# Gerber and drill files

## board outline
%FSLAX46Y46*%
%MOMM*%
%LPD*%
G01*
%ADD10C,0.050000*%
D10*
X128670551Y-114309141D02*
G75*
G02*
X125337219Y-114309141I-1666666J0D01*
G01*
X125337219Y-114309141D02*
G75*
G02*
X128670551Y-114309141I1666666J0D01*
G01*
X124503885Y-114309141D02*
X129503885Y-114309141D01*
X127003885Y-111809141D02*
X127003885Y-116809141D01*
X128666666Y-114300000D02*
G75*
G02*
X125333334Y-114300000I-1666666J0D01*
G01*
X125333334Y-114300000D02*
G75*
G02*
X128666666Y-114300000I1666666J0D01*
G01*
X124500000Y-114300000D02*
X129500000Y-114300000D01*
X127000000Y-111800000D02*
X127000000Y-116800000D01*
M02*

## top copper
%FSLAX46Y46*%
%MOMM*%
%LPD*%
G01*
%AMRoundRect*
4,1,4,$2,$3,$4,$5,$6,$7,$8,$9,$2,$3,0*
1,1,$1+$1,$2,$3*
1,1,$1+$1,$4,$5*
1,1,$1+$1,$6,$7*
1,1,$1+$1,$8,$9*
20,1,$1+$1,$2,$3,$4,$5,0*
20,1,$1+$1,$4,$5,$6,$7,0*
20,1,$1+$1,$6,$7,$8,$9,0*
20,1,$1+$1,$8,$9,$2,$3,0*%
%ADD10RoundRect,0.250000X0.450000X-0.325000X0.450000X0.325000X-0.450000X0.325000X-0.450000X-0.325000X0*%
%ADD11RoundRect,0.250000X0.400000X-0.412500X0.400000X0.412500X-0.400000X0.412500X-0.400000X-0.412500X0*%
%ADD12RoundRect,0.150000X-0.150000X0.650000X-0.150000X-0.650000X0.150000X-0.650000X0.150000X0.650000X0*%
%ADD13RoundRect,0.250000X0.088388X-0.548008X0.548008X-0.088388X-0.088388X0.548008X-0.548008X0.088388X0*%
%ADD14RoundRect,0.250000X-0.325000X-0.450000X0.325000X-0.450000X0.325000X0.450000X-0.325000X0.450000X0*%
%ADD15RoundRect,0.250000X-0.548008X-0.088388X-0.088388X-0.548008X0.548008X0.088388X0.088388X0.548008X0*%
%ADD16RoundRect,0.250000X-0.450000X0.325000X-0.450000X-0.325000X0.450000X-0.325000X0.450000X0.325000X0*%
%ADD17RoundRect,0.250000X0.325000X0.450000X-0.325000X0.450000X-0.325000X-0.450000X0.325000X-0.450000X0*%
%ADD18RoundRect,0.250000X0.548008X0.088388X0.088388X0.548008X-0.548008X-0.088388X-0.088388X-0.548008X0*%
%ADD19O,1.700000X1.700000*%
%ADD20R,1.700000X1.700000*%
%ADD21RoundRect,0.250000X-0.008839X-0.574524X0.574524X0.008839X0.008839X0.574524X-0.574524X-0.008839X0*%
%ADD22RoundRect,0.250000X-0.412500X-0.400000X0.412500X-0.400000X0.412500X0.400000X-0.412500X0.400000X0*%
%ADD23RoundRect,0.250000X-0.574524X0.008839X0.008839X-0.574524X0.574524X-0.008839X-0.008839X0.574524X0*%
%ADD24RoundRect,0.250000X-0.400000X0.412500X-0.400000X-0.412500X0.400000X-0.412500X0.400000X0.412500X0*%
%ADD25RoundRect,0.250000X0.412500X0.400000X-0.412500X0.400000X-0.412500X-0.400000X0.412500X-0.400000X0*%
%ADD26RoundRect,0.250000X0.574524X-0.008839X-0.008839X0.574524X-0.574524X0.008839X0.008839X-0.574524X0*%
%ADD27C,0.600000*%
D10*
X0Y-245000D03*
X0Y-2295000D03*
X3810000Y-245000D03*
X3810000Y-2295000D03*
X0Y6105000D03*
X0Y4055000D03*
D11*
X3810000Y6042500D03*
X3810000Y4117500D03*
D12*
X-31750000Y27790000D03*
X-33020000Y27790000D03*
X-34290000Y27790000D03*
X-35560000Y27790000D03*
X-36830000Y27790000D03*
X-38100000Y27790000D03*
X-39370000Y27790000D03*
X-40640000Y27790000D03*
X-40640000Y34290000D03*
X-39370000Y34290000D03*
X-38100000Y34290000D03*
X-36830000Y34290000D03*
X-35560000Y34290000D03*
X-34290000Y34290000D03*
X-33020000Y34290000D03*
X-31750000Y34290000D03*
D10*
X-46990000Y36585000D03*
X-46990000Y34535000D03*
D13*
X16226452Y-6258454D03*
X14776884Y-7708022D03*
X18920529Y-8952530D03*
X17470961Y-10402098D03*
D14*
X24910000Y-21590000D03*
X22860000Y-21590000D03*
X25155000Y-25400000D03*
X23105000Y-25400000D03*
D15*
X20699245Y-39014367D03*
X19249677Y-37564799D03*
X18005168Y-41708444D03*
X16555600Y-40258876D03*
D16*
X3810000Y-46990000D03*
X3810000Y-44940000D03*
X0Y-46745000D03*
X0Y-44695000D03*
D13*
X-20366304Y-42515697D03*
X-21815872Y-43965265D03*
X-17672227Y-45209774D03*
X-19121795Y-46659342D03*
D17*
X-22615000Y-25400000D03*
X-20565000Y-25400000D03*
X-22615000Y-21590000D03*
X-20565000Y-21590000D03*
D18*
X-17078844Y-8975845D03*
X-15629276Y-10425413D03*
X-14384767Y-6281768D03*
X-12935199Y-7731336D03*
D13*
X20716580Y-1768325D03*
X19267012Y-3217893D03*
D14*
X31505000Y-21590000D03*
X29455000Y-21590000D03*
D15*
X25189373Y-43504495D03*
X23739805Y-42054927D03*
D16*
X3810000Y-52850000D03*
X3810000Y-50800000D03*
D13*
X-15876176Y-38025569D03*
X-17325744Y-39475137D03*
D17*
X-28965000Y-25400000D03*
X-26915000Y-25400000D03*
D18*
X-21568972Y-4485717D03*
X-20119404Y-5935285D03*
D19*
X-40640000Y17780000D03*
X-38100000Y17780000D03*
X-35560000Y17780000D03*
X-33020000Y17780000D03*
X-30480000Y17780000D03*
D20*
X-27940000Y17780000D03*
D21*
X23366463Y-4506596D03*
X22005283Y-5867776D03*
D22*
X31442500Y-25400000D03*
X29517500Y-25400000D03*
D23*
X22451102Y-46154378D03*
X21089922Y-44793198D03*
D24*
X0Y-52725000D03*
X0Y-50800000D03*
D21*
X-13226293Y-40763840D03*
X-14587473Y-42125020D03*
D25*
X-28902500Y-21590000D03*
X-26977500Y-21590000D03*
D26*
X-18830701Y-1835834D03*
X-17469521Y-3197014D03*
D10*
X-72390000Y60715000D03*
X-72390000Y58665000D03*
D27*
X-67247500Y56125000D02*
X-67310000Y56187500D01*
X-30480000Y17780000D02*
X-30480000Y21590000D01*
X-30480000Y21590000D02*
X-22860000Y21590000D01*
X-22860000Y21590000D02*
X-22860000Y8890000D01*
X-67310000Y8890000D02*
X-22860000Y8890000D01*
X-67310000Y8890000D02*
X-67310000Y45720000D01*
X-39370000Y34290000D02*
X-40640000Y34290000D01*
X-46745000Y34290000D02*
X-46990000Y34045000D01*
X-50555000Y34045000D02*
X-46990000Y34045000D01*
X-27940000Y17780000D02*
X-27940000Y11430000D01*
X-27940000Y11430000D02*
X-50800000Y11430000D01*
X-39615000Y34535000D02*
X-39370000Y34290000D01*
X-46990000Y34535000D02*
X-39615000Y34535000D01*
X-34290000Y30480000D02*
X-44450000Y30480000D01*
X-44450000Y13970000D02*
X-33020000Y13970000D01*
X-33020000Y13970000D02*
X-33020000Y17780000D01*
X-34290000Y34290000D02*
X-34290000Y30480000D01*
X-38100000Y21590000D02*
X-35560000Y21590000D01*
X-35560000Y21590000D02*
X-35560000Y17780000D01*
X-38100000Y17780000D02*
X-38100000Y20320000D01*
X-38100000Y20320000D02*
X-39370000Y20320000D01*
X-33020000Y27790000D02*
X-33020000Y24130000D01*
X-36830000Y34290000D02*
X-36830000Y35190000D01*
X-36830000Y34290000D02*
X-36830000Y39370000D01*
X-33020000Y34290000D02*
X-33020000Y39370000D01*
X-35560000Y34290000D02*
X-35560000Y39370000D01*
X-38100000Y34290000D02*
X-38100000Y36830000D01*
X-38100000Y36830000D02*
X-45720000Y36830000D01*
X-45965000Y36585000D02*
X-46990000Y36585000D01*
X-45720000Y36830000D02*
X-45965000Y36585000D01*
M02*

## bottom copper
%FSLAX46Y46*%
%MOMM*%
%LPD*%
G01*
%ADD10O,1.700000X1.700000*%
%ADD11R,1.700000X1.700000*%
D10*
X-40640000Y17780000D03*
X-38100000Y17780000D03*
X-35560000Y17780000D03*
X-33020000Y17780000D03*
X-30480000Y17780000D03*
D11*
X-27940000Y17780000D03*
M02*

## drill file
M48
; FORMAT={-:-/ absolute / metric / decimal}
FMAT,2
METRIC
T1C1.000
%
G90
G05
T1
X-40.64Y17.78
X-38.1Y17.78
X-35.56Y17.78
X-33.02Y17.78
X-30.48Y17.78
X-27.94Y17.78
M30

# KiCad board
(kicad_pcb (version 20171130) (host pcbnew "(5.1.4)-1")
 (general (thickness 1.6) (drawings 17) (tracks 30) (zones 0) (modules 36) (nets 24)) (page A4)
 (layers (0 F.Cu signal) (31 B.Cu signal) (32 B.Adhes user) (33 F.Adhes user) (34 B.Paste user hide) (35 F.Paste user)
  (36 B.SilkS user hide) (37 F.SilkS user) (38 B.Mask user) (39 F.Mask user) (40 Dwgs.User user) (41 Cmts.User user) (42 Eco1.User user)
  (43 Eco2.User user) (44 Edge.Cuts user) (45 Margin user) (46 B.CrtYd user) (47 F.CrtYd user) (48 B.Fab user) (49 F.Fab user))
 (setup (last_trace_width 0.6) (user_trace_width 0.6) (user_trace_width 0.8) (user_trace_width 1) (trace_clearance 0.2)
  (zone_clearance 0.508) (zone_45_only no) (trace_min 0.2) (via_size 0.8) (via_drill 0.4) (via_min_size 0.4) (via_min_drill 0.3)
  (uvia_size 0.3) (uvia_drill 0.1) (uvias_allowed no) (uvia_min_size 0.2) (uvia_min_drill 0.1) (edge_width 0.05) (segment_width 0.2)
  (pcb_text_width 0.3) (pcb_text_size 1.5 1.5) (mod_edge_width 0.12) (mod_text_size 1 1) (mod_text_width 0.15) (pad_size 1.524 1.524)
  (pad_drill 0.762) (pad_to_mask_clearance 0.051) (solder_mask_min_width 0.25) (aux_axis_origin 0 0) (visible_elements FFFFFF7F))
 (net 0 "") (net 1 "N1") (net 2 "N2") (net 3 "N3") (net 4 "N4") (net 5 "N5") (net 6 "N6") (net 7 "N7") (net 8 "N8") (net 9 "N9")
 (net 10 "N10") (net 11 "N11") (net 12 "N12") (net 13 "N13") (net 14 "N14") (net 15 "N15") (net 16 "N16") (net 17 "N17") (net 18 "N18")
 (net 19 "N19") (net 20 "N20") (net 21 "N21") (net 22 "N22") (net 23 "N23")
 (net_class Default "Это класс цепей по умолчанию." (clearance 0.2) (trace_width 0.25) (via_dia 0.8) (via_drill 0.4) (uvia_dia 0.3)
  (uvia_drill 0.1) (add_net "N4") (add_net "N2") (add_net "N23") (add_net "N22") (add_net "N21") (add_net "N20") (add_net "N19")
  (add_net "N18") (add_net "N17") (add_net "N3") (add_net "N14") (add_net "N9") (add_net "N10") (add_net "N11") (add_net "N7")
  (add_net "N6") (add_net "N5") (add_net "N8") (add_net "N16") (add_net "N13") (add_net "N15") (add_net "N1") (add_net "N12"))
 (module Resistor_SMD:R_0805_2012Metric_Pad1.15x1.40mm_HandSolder (layer F.Cu) (at 0 1.27 90)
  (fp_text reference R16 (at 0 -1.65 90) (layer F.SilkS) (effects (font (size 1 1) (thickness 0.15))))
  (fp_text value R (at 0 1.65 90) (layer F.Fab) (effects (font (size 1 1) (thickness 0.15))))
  (pad 2 smd roundrect (at 1.025 0 90) (size 1.15 1.4) (layers F.Cu F.Paste F.Mask) (roundrect_rratio 0.217391) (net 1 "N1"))
  (pad 1 smd roundrect (at -1.025 0 90) (size 1.15 1.4) (layers F.Cu F.Paste F.Mask) (roundrect_rratio 0.217391) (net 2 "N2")))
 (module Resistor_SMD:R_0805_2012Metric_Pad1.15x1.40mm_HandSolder (layer F.Cu) (at 3.81 1.27 90)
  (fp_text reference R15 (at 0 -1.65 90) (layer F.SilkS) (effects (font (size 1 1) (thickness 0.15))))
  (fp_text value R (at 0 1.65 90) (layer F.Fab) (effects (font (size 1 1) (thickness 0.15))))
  (pad 2 smd roundrect (at 1.025 0 90) (size 1.15 1.4) (layers F.Cu F.Paste F.Mask) (roundrect_rratio 0.217391) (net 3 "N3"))
  (pad 1 smd roundrect (at -1.025 0 90) (size 1.15 1.4) (layers F.Cu F.Paste F.Mask) (roundrect_rratio 0.217391) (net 2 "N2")))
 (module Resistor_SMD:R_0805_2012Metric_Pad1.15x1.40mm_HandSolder (layer F.Cu) (at 0 -5.08 90)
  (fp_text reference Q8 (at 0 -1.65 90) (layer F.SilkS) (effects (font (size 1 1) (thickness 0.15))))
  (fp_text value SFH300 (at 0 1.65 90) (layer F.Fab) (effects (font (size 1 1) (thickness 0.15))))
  (pad 2 smd roundrect (at 1.025 0 90) (size 1.15 1.4) (layers F.Cu F.Paste F.Mask) (roundrect_rratio 0.217391) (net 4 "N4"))
  (pad 1 smd roundrect (at -1.025 0 90) (size 1.15 1.4) (layers F.Cu F.Paste F.Mask) (roundrect_rratio 0.217391) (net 1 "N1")))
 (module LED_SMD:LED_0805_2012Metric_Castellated (layer F.Cu) (at 3.81 -5.08 90)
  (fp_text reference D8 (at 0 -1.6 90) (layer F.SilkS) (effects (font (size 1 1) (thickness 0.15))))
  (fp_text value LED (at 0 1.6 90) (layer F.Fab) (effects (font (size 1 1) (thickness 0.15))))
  (pad 2 smd roundrect (at 0.9625 0 90) (size 1.325 1.3) (layers F.Cu F.Paste F.Mask) (roundrect_rratio 0.192308) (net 4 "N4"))
  (pad 1 smd roundrect (at -0.9625 0 90) (size 1.325 1.3) (layers F.Cu F.Paste F.Mask) (roundrect_rratio 0.192308) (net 3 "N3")))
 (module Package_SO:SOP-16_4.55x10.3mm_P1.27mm (layer F.Cu) (at -36.195 -31.04 270)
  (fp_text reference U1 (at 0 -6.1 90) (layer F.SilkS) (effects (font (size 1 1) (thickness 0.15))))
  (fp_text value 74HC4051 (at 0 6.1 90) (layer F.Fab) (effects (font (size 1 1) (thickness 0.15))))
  (pad 16 smd roundrect (at 3.25 -4.445 270) (size 1.6 0.6) (layers F.Cu F.Paste F.Mask) (roundrect_rratio 0.25) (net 4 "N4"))
  (pad 15 smd roundrect (at 3.25 -3.175 270) (size 1.6 0.6) (layers F.Cu F.Paste F.Mask) (roundrect_rratio 0.25) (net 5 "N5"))
  (pad 14 smd roundrect (at 3.25 -1.905 270) (size 1.6 0.6) (layers F.Cu F.Paste F.Mask) (roundrect_rratio 0.25) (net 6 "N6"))
  (pad 13 smd roundrect (at 3.25 -0.635 270) (size 1.6 0.6) (layers F.Cu F.Paste F.Mask) (roundrect_rratio 0.25) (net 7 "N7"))
  (pad 12 smd roundrect (at 3.25 0.635 270) (size 1.6 0.6) (layers F.Cu F.Paste F.Mask) (roundrect_rratio 0.25) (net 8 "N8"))
  (pad 11 smd roundrect (at 3.25 1.905 270) (size 1.6 0.6) (layers F.Cu F.Paste F.Mask) (roundrect_rratio 0.25) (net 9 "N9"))
  (pad 10 smd roundrect (at 3.25 3.175 270) (size 1.6 0.6) (layers F.Cu F.Paste F.Mask) (roundrect_rratio 0.25) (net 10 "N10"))
  (pad 9 smd roundrect (at 3.25 4.445 270) (size 1.6 0.6) (layers F.Cu F.Paste F.Mask) (roundrect_rratio 0.25) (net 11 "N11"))
  (pad 8 smd roundrect (at -3.25 4.445 270) (size 1.6 0.6) (layers F.Cu F.Paste F.Mask) (roundrect_rratio 0.25) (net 2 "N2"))
  (pad 7 smd roundrect (at -3.25 3.175 270) (size 1.6 0.6) (layers F.Cu F.Paste F.Mask) (roundrect_rratio 0.25) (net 2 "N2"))
  (pad 6 smd roundrect (at -3.25 1.905 270) (size 1.6 0.6) (layers F.Cu F.Paste F.Mask) (roundrect_rratio 0.25) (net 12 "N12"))
  (pad 5 smd roundrect (at -3.25 0.635 270) (size 1.6 0.6) (layers F.Cu F.Paste F.Mask) (roundrect_rratio 0.25) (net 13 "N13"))
  (pad 4 smd roundrect (at -3.25 -0.635 270) (size 1.6 0.6) (layers F.Cu F.Paste F.Mask) (roundrect_rratio 0.25) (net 1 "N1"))
  (pad 3 smd roundrect (at -3.25 -1.905 270) (size 1.6 0.6) (layers F.Cu F.Paste F.Mask) (roundrect_rratio 0.25) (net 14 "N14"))
  (pad 2 smd roundrect (at -3.25 -3.175 270) (size 1.6 0.6) (layers F.Cu F.Paste F.Mask) (roundrect_rratio 0.25) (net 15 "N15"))
  (pad 1 smd roundrect (at -3.25 -4.445 270) (size 1.6 0.6) (layers F.Cu F.Paste F.Mask) (roundrect_rratio 0.25) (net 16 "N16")))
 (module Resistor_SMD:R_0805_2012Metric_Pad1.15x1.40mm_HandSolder (layer F.Cu) (at -46.99 -35.56 90)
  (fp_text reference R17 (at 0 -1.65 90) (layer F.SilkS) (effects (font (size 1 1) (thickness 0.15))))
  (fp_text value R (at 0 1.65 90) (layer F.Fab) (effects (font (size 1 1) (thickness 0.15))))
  (pad 2 smd roundrect (at 1.025 0 90) (size 1.15 1.4) (layers F.Cu F.Paste F.Mask) (roundrect_rratio 0.217391) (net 12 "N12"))
  (pad 1 smd roundrect (at -1.025 0 90) (size 1.15 1.4) (layers F.Cu F.Paste F.Mask) (roundrect_rratio 0.217391) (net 2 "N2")))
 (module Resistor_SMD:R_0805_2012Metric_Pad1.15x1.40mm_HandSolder (layer F.Cu) (at 15.501668 6.983238 45)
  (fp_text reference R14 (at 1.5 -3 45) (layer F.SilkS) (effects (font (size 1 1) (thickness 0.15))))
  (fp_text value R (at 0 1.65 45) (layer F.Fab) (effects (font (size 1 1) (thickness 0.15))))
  (pad 2 smd roundrect (at 1.025 0 45) (size 1.15 1.4) (layers F.Cu F.Paste F.Mask) (roundrect_rratio 0.217391) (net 15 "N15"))
  (pad 1 smd roundrect (at -1.025 0 45) (size 1.15 1.4) (layers F.Cu F.Paste F.Mask) (roundrect_rratio 0.217391) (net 2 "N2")))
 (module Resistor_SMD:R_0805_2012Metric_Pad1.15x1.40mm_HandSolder (layer F.Cu) (at 18.195745 9.677314 45)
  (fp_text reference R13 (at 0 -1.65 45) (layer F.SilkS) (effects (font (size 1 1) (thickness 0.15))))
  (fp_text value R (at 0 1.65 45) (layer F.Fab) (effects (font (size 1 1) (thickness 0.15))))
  (pad 2 smd roundrect (at 1.025 0 45) (size 1.15 1.4) (layers F.Cu F.Paste F.Mask) (roundrect_rratio 0.217391) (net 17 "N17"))
  (pad 1 smd roundrect (at -1.025 0 45) (size 1.15 1.4) (layers F.Cu F.Paste F.Mask) (roundrect_rratio 0.217391) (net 2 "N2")))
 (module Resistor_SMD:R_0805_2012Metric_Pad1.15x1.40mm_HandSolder (layer F.Cu) (at 23.885 21.59)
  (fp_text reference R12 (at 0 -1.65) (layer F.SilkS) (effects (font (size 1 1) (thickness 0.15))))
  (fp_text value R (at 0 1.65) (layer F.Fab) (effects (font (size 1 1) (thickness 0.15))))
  (pad 2 smd roundrect (at 1.025 0) (size 1.15 1.4) (layers F.Cu F.Paste F.Mask) (roundrect_rratio 0.217391) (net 13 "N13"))
  (pad 1 smd roundrect (at -1.025 0) (size 1.15 1.4) (layers F.Cu F.Paste F.Mask) (roundrect_rratio 0.217391) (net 2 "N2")))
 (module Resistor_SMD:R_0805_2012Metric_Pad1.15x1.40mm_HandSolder (layer F.Cu) (at 24.13 25.4)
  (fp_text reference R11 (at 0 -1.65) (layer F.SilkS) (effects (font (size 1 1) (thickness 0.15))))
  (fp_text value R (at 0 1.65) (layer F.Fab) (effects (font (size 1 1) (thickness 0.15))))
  (pad 2 smd roundrect (at 1.025 0) (size 1.15 1.4) (layers F.Cu F.Paste F.Mask) (roundrect_rratio 0.217391) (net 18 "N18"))
  (pad 1 smd roundrect (at -1.025 0) (size 1.15 1.4) (layers F.Cu F.Paste F.Mask) (roundrect_rratio 0.217391) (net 2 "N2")))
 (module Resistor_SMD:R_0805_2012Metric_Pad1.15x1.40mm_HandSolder (layer F.Cu) (at 19.974461 38.289583 315)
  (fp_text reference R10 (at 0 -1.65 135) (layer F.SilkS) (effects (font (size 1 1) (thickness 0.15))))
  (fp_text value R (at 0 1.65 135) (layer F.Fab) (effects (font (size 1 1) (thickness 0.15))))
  (pad 2 smd roundrect (at 1.025 0 315) (size 1.15 1.4) (layers F.Cu F.Paste F.Mask) (roundrect_rratio 0.217391) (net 16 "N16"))
  (pad 1 smd roundrect (at -1.025 0 315) (size 1.15 1.4) (layers F.Cu F.Paste F.Mask) (roundrect_rratio 0.217391) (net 2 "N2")))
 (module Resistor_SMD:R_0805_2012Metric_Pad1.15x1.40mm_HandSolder (layer F.Cu) (at 17.280384 40.98366 315)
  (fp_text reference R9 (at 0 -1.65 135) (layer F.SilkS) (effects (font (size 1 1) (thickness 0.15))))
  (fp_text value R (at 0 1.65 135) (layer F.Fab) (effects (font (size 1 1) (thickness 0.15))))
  (pad 2 smd roundrect (at 1.025 0 315) (size 1.15 1.4) (layers F.Cu F.Paste F.Mask) (roundrect_rratio 0.217391) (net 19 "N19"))
  (pad 1 smd roundrect (at -1.025 0 315) (size 1.15 1.4) (layers F.Cu F.Paste F.Mask) (roundrect_rratio 0.217391) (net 2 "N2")))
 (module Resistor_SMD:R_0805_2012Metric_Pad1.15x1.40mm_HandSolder (layer F.Cu) (at 3.81 45.965 270)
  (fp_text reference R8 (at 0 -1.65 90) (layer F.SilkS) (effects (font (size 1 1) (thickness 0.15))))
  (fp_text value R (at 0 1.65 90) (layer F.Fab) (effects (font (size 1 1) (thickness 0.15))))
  (pad 2 smd roundrect (at 1.025 0 270) (size 1.15 1.4) (layers F.Cu F.Paste F.Mask) (roundrect_rratio 0.217391) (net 8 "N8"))
  (pad 1 smd roundrect (at -1.025 0 270) (size 1.15 1.4) (layers F.Cu F.Paste F.Mask) (roundrect_rratio 0.217391) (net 2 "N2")))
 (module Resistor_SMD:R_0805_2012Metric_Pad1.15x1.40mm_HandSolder (layer F.Cu) (at 0 45.72 270)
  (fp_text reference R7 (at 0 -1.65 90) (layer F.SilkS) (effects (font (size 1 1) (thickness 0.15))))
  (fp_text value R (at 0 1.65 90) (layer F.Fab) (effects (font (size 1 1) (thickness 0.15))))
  (pad 2 smd roundrect (at 1.025 0 270) (size 1.15 1.4) (layers F.Cu F.Paste F.Mask) (roundrect_rratio 0.217391) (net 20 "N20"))
  (pad 1 smd roundrect (at -1.025 0 270) (size 1.15 1.4) (layers F.Cu F.Paste F.Mask) (roundrect_rratio 0.217391) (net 2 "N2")))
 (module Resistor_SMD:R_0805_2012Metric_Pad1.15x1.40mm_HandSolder (layer F.Cu) (at -21.091088 43.240481 45)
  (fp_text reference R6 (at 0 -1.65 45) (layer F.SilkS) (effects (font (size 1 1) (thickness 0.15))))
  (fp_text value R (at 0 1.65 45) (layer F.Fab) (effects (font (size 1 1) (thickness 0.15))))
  (pad 2 smd roundrect (at 1.025 0 45) (size 1.15 1.4) (layers F.Cu F.Paste F.Mask) (roundrect_rratio 0.217391) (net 5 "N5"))
  (pad 1 smd roundrect (at -1.025 0 45) (size 1.15 1.4) (layers F.Cu F.Paste F.Mask) (roundrect_rratio 0.217391) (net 2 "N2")))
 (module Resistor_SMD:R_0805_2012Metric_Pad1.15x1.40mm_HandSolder (layer F.Cu) (at -18.397011 45.934558 45)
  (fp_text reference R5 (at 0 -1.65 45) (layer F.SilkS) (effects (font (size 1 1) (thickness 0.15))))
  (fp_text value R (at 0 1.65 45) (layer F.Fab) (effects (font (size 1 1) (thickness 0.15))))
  (pad 2 smd roundrect (at 1.025 0 45) (size 1.15 1.4) (layers F.Cu F.Paste F.Mask) (roundrect_rratio 0.217391) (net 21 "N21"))
  (pad 1 smd roundrect (at -1.025 0 45) (size 1.15 1.4) (layers F.Cu F.Paste F.Mask) (roundrect_rratio 0.217391) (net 2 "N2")))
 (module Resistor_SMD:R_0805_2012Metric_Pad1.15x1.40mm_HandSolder (layer F.Cu) (at -21.59 25.4 180)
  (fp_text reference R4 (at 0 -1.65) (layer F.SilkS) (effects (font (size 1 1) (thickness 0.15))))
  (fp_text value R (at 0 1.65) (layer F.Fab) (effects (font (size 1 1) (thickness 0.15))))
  (pad 2 smd roundrect (at 1.025 0 180) (size 1.15 1.4) (layers F.Cu F.Paste F.Mask) (roundrect_rratio 0.217391) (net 6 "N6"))
  (pad 1 smd roundrect (at -1.025 0 180) (size 1.15 1.4) (layers F.Cu F.Paste F.Mask) (roundrect_rratio 0.217391) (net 2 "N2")))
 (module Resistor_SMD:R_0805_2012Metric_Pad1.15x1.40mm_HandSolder (layer F.Cu) (at -21.59 21.59 180)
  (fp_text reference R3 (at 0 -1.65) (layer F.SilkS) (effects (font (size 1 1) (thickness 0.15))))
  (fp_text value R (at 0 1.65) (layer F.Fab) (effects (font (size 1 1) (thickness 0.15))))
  (pad 2 smd roundrect (at 1.025 0 180) (size 1.15 1.4) (layers F.Cu F.Paste F.Mask) (roundrect_rratio 0.217391) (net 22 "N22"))
  (pad 1 smd roundrect (at -1.025 0 180) (size 1.15 1.4) (layers F.Cu F.Paste F.Mask) (roundrect_rratio 0.217391) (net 2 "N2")))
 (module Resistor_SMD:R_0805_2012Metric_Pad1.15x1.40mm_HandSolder (layer F.Cu) (at -16.35406 9.700629 135)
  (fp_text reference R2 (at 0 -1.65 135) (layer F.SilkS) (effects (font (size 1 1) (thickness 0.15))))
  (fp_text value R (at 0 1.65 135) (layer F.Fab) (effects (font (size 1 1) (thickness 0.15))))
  (pad 2 smd roundrect (at 1.025 0 135) (size 1.15 1.4) (layers F.Cu F.Paste F.Mask) (roundrect_rratio 0.217391) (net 7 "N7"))
  (pad 1 smd roundrect (at -1.025 0 135) (size 1.15 1.4) (layers F.Cu F.Paste F.Mask) (roundrect_rratio 0.217391) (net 2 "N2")))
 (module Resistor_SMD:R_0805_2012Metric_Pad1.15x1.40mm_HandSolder (layer F.Cu) (at -13.659983 7.006552 135)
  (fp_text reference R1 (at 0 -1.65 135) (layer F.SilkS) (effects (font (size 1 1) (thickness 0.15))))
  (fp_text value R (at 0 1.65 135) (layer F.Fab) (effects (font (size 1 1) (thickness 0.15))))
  (pad 2 smd roundrect (at 1.025 0 135) (size 1.15 1.4) (layers F.Cu F.Paste F.Mask) (roundrect_rratio 0.217391) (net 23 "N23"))
  (pad 1 smd roundrect (at -1.025 0 135) (size 1.15 1.4) (layers F.Cu F.Paste F.Mask) (roundrect_rratio 0.217391) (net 2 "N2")))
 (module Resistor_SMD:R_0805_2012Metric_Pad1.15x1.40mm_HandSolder (layer F.Cu) (at 19.991796 2.493109 45)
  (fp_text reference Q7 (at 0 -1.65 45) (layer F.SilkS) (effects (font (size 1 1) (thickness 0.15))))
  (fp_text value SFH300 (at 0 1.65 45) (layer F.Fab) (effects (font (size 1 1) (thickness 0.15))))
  (pad 2 smd roundrect (at 1.025 0 45) (size 1.15 1.4) (layers F.Cu F.Paste F.Mask) (roundrect_rratio 0.217391) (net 4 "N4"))
  (pad 1 smd roundrect (at -1.025 0 45) (size 1.15 1.4) (layers F.Cu F.Paste F.Mask) (roundrect_rratio 0.217391) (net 15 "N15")))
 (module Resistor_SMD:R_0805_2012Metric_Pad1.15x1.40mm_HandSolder (layer F.Cu) (at 30.48 21.59)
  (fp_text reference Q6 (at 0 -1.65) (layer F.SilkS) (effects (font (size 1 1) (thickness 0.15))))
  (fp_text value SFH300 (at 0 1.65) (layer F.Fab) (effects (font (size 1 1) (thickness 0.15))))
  (pad 2 smd roundrect (at 1.025 0) (size 1.15 1.4) (layers F.Cu F.Paste F.Mask) (roundrect_rratio 0.217391) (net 4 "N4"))
  (pad 1 smd roundrect (at -1.025 0) (size 1.15 1.4) (layers F.Cu F.Paste F.Mask) (roundrect_rratio 0.217391) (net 13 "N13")))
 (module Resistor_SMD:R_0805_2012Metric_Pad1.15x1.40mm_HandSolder (layer F.Cu) (at 24.464589 42.779711 315)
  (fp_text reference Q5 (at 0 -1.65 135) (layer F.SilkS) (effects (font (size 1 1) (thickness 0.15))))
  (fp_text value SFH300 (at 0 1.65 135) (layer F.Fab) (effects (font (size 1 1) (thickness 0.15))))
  (pad 2 smd roundrect (at 1.025 0 315) (size 1.15 1.4) (layers F.Cu F.Paste F.Mask) (roundrect_rratio 0.217391) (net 4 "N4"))
  (pad 1 smd roundrect (at -1.025 0 315) (size 1.15 1.4) (layers F.Cu F.Paste F.Mask) (roundrect_rratio 0.217391) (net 16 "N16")))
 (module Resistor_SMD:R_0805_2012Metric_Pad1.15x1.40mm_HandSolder (layer F.Cu) (at 3.81 51.825 270)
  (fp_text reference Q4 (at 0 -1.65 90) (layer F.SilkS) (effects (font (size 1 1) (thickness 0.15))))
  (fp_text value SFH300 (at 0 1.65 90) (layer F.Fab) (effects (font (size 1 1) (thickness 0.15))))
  (pad 2 smd roundrect (at 1.025 0 270) (size 1.15 1.4) (layers F.Cu F.Paste F.Mask) (roundrect_rratio 0.217391) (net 4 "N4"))
  (pad 1 smd roundrect (at -1.025 0 270) (size 1.15 1.4) (layers F.Cu F.Paste F.Mask) (roundrect_rratio 0.217391) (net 8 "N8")))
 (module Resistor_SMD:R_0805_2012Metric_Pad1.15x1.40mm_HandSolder (layer F.Cu) (at -16.60096 38.750353 45)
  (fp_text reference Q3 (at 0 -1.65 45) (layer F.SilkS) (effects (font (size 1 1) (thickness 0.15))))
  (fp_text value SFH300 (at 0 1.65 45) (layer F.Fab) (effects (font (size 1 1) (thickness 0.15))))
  (pad 2 smd roundrect (at 1.025 0 45) (size 1.15 1.4) (layers F.Cu F.Paste F.Mask) (roundrect_rratio 0.217391) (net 4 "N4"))
  (pad 1 smd roundrect (at -1.025 0 45) (size 1.15 1.4) (layers F.Cu F.Paste F.Mask) (roundrect_rratio 0.217391) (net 5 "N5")))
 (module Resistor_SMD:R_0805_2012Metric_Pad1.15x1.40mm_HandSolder (layer F.Cu) (at -27.94 25.4 180)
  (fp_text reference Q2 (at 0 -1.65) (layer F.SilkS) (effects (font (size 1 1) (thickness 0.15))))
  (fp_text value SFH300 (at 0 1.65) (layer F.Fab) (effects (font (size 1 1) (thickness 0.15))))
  (pad 2 smd roundrect (at 1.025 0 180) (size 1.15 1.4) (layers F.Cu F.Paste F.Mask) (roundrect_rratio 0.217391) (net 4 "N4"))
  (pad 1 smd roundrect (at -1.025 0 180) (size 1.15 1.4) (layers F.Cu F.Paste F.Mask) (roundrect_rratio 0.217391) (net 6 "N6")))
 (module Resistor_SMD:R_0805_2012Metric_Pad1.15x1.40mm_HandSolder (layer F.Cu) (at -20.844188 5.210501 135)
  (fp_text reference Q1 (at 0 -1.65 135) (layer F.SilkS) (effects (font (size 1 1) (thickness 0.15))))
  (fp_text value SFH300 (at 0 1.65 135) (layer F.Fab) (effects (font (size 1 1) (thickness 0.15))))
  (pad 2 smd roundrect (at 1.025 0 135) (size 1.15 1.4) (layers F.Cu F.Paste F.Mask) (roundrect_rratio 0.217391) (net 4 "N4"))
  (pad 1 smd roundrect (at -1.025 0 135) (size 1.15 1.4) (layers F.Cu F.Paste F.Mask) (roundrect_rratio 0.217391) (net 7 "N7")))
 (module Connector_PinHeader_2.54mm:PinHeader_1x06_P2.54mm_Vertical (layer F.Cu) (at -27.94 -17.78 270)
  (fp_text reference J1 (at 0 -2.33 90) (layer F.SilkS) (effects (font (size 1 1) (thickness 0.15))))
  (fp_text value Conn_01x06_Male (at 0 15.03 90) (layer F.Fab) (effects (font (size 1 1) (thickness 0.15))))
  (pad 6 thru_hole oval (at 0 12.7 270) (size 1.7 1.7) (drill 1) (layers *.Cu *.Mask) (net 11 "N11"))
  (pad 5 thru_hole oval (at 0 10.16 270) (size 1.7 1.7) (drill 1) (layers *.Cu *.Mask) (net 10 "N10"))
  (pad 4 thru_hole oval (at 0 7.62 270) (size 1.7 1.7) (drill 1) (layers *.Cu *.Mask) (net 9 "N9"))
  (pad 3 thru_hole oval (at 0 5.08 270) (size 1.7 1.7) (drill 1) (layers *.Cu *.Mask) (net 14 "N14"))
  (pad 2 thru_hole oval (at 0 2.54 270) (size 1.7 1.7) (drill 1) (layers *.Cu *.Mask) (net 4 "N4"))
  (pad 1 thru_hole rect (at 0 0 270) (size 1.7 1.7) (drill 1) (layers *.Cu *.Mask) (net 2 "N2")))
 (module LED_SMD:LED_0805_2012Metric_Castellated (layer F.Cu) (at 22.685873 5.187186 45)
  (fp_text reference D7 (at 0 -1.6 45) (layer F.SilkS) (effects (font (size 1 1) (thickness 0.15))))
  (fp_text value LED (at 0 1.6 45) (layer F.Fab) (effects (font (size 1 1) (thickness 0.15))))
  (pad 2 smd roundrect (at 0.9625 0 45) (size 1.325 1.3) (layers F.Cu F.Paste F.Mask) (roundrect_rratio 0.192308) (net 4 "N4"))
  (pad 1 smd roundrect (at -0.9625 0 45) (size 1.325 1.3) (layers F.Cu F.Paste F.Mask) (roundrect_rratio 0.192308) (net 17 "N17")))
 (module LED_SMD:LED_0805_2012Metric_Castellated (layer F.Cu) (at 30.48 25.4)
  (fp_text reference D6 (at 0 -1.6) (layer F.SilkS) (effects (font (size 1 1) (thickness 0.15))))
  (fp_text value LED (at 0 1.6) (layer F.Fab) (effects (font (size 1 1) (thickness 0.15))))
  (pad 2 smd roundrect (at 0.9625 0) (size 1.325 1.3) (layers F.Cu F.Paste F.Mask) (roundrect_rratio 0.192308) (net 4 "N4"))
  (pad 1 smd roundrect (at -0.9625 0) (size 1.325 1.3) (layers F.Cu F.Paste F.Mask) (roundrect_rratio 0.192308) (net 18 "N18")))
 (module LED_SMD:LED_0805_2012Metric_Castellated (layer F.Cu) (at 21.770512 45.473788 315)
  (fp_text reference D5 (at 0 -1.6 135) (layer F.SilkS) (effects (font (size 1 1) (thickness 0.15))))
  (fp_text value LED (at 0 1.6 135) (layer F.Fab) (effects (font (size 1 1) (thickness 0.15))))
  (pad 2 smd roundrect (at 0.9625 0 315) (size 1.325 1.3) (layers F.Cu F.Paste F.Mask) (roundrect_rratio 0.192308) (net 4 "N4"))
  (pad 1 smd roundrect (at -0.9625 0 315) (size 1.325 1.3) (layers F.Cu F.Paste F.Mask) (roundrect_rratio 0.192308) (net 19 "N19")))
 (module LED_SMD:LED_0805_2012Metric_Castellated (layer F.Cu) (at 0 51.7625 270)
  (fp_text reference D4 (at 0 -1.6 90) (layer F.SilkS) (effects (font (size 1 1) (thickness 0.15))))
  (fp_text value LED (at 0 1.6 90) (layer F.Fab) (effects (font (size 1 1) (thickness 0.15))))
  (pad 2 smd roundrect (at 0.9625 0 270) (size 1.325 1.3) (layers F.Cu F.Paste F.Mask) (roundrect_rratio 0.192308) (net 4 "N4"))
  (pad 1 smd roundrect (at -0.9625 0 270) (size 1.325 1.3) (layers F.Cu F.Paste F.Mask) (roundrect_rratio 0.192308) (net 20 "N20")))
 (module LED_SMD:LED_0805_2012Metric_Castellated (layer F.Cu) (at -13.906883 41.44443 45)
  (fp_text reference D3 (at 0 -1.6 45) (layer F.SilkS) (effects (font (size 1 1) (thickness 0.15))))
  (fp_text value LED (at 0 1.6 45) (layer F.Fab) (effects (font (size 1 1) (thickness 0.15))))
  (pad 2 smd roundrect (at 0.9625 0 45) (size 1.325 1.3) (layers F.Cu F.Paste F.Mask) (roundrect_rratio 0.192308) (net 4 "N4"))
  (pad 1 smd roundrect (at -0.9625 0 45) (size 1.325 1.3) (layers F.Cu F.Paste F.Mask) (roundrect_rratio 0.192308) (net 21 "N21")))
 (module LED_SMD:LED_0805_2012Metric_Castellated (layer F.Cu) (at -27.94 21.59 180)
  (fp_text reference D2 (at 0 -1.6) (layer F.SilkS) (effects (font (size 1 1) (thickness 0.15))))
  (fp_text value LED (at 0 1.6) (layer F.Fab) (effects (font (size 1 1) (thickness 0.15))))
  (pad 2 smd roundrect (at 0.9625 0 180) (size 1.325 1.3) (layers F.Cu F.Paste F.Mask) (roundrect_rratio 0.192308) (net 4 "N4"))
  (pad 1 smd roundrect (at -0.9625 0 180) (size 1.325 1.3) (layers F.Cu F.Paste F.Mask) (roundrect_rratio 0.192308) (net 22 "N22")))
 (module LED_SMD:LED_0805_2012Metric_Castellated (layer F.Cu) (at -18.150111 2.516424 135)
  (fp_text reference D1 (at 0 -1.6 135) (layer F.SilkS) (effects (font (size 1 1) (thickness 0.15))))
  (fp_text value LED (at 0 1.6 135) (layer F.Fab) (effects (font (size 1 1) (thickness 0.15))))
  (pad 2 smd roundrect (at 0.9625 0 135) (size 1.325 1.3) (layers F.Cu F.Paste F.Mask) (roundrect_rratio 0.192308) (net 4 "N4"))
  (pad 1 smd roundrect (at -0.9625 0 135) (size 1.325 1.3) (layers F.Cu F.Paste F.Mask) (roundrect_rratio 0.192308) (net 23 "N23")))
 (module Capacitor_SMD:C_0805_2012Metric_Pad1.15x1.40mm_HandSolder (layer F.Cu) (at -72.39 -59.69 90)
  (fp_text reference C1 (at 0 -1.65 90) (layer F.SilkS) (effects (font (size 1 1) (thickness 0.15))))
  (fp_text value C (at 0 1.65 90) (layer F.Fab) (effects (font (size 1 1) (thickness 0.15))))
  (pad 2 smd roundrect (at 1.025 0 90) (size 1.15 1.4) (layers F.Cu F.Paste F.Mask) (roundrect_rratio 0.217391) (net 2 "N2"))
  (pad 1 smd roundrect (at -1.025 0 90) (size 1.15 1.4) (layers F.Cu F.Paste F.Mask) (roundrect_rratio 0.217391) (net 4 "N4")))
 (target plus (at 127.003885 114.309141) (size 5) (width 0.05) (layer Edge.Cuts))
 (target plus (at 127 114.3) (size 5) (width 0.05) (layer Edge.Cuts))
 (segment (start -67.2475 -56.125) (end -67.31 -56.1875) (width 0.6) (layer F.Cu) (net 4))
 (segment (start -30.48 -17.78) (end -30.48 -21.59) (width 0.6) (layer F.Cu) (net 4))
 (segment (start -30.48 -21.59) (end -22.86 -21.59) (width 0.6) (layer F.Cu) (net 4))
 (segment (start -22.86 -21.59) (end -22.86 -8.89) (width 0.6) (layer F.Cu) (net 4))
 (segment (start -67.31 -8.89) (end -22.86 -8.89) (width 0.6) (layer F.Cu) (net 4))
 (segment (start -67.31 -8.89) (end -67.31 -45.72) (width 0.6) (layer F.Cu) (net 4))
 (segment (start -39.37 -34.29) (end -40.64 -34.29) (width 0.6) (layer F.Cu) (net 2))
 (segment (start -46.745 -34.29) (end -46.99 -34.045) (width 0.6) (layer F.Cu) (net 2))
 (segment (start -50.555 -34.045) (end -46.99 -34.045) (width 0.6) (layer F.Cu) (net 2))
 (segment (start -27.94 -17.78) (end -27.94 -11.43) (width 0.6) (layer F.Cu) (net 2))
 (segment (start -27.94 -11.43) (end -50.8 -11.43) (width 0.6) (layer F.Cu) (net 2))
 (segment (start -39.615 -34.535) (end -39.37 -34.29) (width 0.6) (layer F.Cu) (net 2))
 (segment (start -46.99 -34.535) (end -39.615 -34.535) (width 0.6) (layer F.Cu) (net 2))
 (segment (start -34.29 -30.48) (end -44.45 -30.48) (width 0.6) (layer F.Cu) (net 14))
 (segment (start -44.45 -13.97) (end -33.02 -13.97) (width 0.6) (layer F.Cu) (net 14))
 (segment (start -33.02 -13.97) (end -33.02 -17.78) (width 0.6) (layer F.Cu) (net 14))
 (segment (start -34.29 -34.29) (end -34.29 -30.48) (width 0.6) (layer F.Cu) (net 14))
 (segment (start -38.1 -21.59) (end -35.56 -21.59) (width 0.6) (layer F.Cu) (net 9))
 (segment (start -35.56 -21.59) (end -35.56 -17.78) (width 0.6) (layer F.Cu) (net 9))
 (segment (start -38.1 -17.78) (end -38.1 -20.32) (width 0.6) (layer F.Cu) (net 10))
 (segment (start -38.1 -20.32) (end -39.37 -20.32) (width 0.6) (layer F.Cu) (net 10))
 (segment (start -33.02 -27.79) (end -33.02 -24.13) (width 0.6) (layer F.Cu) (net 5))
 (segment (start -36.83 -34.29) (end -36.83 -35.19) (width 0.6) (layer F.Cu) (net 13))
 (segment (start -36.83 -34.29) (end -36.83 -39.37) (width 0.6) (layer F.Cu) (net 13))
 (segment (start -33.02 -34.29) (end -33.02 -39.37) (width 0.6) (layer F.Cu) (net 15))
 (segment (start -35.56 -34.29) (end -35.56 -39.37) (width 0.6) (layer F.Cu) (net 1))
 (segment (start -38.1 -34.29) (end -38.1 -36.83) (width 0.6) (layer F.Cu) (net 12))
 (segment (start -38.1 -36.83) (end -45.72 -36.83) (width 0.6) (layer F.Cu) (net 12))
 (segment (start -45.965 -36.585) (end -46.99 -36.585) (width 0.6) (layer F.Cu) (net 12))
 (segment (start -45.72 -36.83) (end -45.965 -36.585) (width 0.6) (layer F.Cu) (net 12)))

